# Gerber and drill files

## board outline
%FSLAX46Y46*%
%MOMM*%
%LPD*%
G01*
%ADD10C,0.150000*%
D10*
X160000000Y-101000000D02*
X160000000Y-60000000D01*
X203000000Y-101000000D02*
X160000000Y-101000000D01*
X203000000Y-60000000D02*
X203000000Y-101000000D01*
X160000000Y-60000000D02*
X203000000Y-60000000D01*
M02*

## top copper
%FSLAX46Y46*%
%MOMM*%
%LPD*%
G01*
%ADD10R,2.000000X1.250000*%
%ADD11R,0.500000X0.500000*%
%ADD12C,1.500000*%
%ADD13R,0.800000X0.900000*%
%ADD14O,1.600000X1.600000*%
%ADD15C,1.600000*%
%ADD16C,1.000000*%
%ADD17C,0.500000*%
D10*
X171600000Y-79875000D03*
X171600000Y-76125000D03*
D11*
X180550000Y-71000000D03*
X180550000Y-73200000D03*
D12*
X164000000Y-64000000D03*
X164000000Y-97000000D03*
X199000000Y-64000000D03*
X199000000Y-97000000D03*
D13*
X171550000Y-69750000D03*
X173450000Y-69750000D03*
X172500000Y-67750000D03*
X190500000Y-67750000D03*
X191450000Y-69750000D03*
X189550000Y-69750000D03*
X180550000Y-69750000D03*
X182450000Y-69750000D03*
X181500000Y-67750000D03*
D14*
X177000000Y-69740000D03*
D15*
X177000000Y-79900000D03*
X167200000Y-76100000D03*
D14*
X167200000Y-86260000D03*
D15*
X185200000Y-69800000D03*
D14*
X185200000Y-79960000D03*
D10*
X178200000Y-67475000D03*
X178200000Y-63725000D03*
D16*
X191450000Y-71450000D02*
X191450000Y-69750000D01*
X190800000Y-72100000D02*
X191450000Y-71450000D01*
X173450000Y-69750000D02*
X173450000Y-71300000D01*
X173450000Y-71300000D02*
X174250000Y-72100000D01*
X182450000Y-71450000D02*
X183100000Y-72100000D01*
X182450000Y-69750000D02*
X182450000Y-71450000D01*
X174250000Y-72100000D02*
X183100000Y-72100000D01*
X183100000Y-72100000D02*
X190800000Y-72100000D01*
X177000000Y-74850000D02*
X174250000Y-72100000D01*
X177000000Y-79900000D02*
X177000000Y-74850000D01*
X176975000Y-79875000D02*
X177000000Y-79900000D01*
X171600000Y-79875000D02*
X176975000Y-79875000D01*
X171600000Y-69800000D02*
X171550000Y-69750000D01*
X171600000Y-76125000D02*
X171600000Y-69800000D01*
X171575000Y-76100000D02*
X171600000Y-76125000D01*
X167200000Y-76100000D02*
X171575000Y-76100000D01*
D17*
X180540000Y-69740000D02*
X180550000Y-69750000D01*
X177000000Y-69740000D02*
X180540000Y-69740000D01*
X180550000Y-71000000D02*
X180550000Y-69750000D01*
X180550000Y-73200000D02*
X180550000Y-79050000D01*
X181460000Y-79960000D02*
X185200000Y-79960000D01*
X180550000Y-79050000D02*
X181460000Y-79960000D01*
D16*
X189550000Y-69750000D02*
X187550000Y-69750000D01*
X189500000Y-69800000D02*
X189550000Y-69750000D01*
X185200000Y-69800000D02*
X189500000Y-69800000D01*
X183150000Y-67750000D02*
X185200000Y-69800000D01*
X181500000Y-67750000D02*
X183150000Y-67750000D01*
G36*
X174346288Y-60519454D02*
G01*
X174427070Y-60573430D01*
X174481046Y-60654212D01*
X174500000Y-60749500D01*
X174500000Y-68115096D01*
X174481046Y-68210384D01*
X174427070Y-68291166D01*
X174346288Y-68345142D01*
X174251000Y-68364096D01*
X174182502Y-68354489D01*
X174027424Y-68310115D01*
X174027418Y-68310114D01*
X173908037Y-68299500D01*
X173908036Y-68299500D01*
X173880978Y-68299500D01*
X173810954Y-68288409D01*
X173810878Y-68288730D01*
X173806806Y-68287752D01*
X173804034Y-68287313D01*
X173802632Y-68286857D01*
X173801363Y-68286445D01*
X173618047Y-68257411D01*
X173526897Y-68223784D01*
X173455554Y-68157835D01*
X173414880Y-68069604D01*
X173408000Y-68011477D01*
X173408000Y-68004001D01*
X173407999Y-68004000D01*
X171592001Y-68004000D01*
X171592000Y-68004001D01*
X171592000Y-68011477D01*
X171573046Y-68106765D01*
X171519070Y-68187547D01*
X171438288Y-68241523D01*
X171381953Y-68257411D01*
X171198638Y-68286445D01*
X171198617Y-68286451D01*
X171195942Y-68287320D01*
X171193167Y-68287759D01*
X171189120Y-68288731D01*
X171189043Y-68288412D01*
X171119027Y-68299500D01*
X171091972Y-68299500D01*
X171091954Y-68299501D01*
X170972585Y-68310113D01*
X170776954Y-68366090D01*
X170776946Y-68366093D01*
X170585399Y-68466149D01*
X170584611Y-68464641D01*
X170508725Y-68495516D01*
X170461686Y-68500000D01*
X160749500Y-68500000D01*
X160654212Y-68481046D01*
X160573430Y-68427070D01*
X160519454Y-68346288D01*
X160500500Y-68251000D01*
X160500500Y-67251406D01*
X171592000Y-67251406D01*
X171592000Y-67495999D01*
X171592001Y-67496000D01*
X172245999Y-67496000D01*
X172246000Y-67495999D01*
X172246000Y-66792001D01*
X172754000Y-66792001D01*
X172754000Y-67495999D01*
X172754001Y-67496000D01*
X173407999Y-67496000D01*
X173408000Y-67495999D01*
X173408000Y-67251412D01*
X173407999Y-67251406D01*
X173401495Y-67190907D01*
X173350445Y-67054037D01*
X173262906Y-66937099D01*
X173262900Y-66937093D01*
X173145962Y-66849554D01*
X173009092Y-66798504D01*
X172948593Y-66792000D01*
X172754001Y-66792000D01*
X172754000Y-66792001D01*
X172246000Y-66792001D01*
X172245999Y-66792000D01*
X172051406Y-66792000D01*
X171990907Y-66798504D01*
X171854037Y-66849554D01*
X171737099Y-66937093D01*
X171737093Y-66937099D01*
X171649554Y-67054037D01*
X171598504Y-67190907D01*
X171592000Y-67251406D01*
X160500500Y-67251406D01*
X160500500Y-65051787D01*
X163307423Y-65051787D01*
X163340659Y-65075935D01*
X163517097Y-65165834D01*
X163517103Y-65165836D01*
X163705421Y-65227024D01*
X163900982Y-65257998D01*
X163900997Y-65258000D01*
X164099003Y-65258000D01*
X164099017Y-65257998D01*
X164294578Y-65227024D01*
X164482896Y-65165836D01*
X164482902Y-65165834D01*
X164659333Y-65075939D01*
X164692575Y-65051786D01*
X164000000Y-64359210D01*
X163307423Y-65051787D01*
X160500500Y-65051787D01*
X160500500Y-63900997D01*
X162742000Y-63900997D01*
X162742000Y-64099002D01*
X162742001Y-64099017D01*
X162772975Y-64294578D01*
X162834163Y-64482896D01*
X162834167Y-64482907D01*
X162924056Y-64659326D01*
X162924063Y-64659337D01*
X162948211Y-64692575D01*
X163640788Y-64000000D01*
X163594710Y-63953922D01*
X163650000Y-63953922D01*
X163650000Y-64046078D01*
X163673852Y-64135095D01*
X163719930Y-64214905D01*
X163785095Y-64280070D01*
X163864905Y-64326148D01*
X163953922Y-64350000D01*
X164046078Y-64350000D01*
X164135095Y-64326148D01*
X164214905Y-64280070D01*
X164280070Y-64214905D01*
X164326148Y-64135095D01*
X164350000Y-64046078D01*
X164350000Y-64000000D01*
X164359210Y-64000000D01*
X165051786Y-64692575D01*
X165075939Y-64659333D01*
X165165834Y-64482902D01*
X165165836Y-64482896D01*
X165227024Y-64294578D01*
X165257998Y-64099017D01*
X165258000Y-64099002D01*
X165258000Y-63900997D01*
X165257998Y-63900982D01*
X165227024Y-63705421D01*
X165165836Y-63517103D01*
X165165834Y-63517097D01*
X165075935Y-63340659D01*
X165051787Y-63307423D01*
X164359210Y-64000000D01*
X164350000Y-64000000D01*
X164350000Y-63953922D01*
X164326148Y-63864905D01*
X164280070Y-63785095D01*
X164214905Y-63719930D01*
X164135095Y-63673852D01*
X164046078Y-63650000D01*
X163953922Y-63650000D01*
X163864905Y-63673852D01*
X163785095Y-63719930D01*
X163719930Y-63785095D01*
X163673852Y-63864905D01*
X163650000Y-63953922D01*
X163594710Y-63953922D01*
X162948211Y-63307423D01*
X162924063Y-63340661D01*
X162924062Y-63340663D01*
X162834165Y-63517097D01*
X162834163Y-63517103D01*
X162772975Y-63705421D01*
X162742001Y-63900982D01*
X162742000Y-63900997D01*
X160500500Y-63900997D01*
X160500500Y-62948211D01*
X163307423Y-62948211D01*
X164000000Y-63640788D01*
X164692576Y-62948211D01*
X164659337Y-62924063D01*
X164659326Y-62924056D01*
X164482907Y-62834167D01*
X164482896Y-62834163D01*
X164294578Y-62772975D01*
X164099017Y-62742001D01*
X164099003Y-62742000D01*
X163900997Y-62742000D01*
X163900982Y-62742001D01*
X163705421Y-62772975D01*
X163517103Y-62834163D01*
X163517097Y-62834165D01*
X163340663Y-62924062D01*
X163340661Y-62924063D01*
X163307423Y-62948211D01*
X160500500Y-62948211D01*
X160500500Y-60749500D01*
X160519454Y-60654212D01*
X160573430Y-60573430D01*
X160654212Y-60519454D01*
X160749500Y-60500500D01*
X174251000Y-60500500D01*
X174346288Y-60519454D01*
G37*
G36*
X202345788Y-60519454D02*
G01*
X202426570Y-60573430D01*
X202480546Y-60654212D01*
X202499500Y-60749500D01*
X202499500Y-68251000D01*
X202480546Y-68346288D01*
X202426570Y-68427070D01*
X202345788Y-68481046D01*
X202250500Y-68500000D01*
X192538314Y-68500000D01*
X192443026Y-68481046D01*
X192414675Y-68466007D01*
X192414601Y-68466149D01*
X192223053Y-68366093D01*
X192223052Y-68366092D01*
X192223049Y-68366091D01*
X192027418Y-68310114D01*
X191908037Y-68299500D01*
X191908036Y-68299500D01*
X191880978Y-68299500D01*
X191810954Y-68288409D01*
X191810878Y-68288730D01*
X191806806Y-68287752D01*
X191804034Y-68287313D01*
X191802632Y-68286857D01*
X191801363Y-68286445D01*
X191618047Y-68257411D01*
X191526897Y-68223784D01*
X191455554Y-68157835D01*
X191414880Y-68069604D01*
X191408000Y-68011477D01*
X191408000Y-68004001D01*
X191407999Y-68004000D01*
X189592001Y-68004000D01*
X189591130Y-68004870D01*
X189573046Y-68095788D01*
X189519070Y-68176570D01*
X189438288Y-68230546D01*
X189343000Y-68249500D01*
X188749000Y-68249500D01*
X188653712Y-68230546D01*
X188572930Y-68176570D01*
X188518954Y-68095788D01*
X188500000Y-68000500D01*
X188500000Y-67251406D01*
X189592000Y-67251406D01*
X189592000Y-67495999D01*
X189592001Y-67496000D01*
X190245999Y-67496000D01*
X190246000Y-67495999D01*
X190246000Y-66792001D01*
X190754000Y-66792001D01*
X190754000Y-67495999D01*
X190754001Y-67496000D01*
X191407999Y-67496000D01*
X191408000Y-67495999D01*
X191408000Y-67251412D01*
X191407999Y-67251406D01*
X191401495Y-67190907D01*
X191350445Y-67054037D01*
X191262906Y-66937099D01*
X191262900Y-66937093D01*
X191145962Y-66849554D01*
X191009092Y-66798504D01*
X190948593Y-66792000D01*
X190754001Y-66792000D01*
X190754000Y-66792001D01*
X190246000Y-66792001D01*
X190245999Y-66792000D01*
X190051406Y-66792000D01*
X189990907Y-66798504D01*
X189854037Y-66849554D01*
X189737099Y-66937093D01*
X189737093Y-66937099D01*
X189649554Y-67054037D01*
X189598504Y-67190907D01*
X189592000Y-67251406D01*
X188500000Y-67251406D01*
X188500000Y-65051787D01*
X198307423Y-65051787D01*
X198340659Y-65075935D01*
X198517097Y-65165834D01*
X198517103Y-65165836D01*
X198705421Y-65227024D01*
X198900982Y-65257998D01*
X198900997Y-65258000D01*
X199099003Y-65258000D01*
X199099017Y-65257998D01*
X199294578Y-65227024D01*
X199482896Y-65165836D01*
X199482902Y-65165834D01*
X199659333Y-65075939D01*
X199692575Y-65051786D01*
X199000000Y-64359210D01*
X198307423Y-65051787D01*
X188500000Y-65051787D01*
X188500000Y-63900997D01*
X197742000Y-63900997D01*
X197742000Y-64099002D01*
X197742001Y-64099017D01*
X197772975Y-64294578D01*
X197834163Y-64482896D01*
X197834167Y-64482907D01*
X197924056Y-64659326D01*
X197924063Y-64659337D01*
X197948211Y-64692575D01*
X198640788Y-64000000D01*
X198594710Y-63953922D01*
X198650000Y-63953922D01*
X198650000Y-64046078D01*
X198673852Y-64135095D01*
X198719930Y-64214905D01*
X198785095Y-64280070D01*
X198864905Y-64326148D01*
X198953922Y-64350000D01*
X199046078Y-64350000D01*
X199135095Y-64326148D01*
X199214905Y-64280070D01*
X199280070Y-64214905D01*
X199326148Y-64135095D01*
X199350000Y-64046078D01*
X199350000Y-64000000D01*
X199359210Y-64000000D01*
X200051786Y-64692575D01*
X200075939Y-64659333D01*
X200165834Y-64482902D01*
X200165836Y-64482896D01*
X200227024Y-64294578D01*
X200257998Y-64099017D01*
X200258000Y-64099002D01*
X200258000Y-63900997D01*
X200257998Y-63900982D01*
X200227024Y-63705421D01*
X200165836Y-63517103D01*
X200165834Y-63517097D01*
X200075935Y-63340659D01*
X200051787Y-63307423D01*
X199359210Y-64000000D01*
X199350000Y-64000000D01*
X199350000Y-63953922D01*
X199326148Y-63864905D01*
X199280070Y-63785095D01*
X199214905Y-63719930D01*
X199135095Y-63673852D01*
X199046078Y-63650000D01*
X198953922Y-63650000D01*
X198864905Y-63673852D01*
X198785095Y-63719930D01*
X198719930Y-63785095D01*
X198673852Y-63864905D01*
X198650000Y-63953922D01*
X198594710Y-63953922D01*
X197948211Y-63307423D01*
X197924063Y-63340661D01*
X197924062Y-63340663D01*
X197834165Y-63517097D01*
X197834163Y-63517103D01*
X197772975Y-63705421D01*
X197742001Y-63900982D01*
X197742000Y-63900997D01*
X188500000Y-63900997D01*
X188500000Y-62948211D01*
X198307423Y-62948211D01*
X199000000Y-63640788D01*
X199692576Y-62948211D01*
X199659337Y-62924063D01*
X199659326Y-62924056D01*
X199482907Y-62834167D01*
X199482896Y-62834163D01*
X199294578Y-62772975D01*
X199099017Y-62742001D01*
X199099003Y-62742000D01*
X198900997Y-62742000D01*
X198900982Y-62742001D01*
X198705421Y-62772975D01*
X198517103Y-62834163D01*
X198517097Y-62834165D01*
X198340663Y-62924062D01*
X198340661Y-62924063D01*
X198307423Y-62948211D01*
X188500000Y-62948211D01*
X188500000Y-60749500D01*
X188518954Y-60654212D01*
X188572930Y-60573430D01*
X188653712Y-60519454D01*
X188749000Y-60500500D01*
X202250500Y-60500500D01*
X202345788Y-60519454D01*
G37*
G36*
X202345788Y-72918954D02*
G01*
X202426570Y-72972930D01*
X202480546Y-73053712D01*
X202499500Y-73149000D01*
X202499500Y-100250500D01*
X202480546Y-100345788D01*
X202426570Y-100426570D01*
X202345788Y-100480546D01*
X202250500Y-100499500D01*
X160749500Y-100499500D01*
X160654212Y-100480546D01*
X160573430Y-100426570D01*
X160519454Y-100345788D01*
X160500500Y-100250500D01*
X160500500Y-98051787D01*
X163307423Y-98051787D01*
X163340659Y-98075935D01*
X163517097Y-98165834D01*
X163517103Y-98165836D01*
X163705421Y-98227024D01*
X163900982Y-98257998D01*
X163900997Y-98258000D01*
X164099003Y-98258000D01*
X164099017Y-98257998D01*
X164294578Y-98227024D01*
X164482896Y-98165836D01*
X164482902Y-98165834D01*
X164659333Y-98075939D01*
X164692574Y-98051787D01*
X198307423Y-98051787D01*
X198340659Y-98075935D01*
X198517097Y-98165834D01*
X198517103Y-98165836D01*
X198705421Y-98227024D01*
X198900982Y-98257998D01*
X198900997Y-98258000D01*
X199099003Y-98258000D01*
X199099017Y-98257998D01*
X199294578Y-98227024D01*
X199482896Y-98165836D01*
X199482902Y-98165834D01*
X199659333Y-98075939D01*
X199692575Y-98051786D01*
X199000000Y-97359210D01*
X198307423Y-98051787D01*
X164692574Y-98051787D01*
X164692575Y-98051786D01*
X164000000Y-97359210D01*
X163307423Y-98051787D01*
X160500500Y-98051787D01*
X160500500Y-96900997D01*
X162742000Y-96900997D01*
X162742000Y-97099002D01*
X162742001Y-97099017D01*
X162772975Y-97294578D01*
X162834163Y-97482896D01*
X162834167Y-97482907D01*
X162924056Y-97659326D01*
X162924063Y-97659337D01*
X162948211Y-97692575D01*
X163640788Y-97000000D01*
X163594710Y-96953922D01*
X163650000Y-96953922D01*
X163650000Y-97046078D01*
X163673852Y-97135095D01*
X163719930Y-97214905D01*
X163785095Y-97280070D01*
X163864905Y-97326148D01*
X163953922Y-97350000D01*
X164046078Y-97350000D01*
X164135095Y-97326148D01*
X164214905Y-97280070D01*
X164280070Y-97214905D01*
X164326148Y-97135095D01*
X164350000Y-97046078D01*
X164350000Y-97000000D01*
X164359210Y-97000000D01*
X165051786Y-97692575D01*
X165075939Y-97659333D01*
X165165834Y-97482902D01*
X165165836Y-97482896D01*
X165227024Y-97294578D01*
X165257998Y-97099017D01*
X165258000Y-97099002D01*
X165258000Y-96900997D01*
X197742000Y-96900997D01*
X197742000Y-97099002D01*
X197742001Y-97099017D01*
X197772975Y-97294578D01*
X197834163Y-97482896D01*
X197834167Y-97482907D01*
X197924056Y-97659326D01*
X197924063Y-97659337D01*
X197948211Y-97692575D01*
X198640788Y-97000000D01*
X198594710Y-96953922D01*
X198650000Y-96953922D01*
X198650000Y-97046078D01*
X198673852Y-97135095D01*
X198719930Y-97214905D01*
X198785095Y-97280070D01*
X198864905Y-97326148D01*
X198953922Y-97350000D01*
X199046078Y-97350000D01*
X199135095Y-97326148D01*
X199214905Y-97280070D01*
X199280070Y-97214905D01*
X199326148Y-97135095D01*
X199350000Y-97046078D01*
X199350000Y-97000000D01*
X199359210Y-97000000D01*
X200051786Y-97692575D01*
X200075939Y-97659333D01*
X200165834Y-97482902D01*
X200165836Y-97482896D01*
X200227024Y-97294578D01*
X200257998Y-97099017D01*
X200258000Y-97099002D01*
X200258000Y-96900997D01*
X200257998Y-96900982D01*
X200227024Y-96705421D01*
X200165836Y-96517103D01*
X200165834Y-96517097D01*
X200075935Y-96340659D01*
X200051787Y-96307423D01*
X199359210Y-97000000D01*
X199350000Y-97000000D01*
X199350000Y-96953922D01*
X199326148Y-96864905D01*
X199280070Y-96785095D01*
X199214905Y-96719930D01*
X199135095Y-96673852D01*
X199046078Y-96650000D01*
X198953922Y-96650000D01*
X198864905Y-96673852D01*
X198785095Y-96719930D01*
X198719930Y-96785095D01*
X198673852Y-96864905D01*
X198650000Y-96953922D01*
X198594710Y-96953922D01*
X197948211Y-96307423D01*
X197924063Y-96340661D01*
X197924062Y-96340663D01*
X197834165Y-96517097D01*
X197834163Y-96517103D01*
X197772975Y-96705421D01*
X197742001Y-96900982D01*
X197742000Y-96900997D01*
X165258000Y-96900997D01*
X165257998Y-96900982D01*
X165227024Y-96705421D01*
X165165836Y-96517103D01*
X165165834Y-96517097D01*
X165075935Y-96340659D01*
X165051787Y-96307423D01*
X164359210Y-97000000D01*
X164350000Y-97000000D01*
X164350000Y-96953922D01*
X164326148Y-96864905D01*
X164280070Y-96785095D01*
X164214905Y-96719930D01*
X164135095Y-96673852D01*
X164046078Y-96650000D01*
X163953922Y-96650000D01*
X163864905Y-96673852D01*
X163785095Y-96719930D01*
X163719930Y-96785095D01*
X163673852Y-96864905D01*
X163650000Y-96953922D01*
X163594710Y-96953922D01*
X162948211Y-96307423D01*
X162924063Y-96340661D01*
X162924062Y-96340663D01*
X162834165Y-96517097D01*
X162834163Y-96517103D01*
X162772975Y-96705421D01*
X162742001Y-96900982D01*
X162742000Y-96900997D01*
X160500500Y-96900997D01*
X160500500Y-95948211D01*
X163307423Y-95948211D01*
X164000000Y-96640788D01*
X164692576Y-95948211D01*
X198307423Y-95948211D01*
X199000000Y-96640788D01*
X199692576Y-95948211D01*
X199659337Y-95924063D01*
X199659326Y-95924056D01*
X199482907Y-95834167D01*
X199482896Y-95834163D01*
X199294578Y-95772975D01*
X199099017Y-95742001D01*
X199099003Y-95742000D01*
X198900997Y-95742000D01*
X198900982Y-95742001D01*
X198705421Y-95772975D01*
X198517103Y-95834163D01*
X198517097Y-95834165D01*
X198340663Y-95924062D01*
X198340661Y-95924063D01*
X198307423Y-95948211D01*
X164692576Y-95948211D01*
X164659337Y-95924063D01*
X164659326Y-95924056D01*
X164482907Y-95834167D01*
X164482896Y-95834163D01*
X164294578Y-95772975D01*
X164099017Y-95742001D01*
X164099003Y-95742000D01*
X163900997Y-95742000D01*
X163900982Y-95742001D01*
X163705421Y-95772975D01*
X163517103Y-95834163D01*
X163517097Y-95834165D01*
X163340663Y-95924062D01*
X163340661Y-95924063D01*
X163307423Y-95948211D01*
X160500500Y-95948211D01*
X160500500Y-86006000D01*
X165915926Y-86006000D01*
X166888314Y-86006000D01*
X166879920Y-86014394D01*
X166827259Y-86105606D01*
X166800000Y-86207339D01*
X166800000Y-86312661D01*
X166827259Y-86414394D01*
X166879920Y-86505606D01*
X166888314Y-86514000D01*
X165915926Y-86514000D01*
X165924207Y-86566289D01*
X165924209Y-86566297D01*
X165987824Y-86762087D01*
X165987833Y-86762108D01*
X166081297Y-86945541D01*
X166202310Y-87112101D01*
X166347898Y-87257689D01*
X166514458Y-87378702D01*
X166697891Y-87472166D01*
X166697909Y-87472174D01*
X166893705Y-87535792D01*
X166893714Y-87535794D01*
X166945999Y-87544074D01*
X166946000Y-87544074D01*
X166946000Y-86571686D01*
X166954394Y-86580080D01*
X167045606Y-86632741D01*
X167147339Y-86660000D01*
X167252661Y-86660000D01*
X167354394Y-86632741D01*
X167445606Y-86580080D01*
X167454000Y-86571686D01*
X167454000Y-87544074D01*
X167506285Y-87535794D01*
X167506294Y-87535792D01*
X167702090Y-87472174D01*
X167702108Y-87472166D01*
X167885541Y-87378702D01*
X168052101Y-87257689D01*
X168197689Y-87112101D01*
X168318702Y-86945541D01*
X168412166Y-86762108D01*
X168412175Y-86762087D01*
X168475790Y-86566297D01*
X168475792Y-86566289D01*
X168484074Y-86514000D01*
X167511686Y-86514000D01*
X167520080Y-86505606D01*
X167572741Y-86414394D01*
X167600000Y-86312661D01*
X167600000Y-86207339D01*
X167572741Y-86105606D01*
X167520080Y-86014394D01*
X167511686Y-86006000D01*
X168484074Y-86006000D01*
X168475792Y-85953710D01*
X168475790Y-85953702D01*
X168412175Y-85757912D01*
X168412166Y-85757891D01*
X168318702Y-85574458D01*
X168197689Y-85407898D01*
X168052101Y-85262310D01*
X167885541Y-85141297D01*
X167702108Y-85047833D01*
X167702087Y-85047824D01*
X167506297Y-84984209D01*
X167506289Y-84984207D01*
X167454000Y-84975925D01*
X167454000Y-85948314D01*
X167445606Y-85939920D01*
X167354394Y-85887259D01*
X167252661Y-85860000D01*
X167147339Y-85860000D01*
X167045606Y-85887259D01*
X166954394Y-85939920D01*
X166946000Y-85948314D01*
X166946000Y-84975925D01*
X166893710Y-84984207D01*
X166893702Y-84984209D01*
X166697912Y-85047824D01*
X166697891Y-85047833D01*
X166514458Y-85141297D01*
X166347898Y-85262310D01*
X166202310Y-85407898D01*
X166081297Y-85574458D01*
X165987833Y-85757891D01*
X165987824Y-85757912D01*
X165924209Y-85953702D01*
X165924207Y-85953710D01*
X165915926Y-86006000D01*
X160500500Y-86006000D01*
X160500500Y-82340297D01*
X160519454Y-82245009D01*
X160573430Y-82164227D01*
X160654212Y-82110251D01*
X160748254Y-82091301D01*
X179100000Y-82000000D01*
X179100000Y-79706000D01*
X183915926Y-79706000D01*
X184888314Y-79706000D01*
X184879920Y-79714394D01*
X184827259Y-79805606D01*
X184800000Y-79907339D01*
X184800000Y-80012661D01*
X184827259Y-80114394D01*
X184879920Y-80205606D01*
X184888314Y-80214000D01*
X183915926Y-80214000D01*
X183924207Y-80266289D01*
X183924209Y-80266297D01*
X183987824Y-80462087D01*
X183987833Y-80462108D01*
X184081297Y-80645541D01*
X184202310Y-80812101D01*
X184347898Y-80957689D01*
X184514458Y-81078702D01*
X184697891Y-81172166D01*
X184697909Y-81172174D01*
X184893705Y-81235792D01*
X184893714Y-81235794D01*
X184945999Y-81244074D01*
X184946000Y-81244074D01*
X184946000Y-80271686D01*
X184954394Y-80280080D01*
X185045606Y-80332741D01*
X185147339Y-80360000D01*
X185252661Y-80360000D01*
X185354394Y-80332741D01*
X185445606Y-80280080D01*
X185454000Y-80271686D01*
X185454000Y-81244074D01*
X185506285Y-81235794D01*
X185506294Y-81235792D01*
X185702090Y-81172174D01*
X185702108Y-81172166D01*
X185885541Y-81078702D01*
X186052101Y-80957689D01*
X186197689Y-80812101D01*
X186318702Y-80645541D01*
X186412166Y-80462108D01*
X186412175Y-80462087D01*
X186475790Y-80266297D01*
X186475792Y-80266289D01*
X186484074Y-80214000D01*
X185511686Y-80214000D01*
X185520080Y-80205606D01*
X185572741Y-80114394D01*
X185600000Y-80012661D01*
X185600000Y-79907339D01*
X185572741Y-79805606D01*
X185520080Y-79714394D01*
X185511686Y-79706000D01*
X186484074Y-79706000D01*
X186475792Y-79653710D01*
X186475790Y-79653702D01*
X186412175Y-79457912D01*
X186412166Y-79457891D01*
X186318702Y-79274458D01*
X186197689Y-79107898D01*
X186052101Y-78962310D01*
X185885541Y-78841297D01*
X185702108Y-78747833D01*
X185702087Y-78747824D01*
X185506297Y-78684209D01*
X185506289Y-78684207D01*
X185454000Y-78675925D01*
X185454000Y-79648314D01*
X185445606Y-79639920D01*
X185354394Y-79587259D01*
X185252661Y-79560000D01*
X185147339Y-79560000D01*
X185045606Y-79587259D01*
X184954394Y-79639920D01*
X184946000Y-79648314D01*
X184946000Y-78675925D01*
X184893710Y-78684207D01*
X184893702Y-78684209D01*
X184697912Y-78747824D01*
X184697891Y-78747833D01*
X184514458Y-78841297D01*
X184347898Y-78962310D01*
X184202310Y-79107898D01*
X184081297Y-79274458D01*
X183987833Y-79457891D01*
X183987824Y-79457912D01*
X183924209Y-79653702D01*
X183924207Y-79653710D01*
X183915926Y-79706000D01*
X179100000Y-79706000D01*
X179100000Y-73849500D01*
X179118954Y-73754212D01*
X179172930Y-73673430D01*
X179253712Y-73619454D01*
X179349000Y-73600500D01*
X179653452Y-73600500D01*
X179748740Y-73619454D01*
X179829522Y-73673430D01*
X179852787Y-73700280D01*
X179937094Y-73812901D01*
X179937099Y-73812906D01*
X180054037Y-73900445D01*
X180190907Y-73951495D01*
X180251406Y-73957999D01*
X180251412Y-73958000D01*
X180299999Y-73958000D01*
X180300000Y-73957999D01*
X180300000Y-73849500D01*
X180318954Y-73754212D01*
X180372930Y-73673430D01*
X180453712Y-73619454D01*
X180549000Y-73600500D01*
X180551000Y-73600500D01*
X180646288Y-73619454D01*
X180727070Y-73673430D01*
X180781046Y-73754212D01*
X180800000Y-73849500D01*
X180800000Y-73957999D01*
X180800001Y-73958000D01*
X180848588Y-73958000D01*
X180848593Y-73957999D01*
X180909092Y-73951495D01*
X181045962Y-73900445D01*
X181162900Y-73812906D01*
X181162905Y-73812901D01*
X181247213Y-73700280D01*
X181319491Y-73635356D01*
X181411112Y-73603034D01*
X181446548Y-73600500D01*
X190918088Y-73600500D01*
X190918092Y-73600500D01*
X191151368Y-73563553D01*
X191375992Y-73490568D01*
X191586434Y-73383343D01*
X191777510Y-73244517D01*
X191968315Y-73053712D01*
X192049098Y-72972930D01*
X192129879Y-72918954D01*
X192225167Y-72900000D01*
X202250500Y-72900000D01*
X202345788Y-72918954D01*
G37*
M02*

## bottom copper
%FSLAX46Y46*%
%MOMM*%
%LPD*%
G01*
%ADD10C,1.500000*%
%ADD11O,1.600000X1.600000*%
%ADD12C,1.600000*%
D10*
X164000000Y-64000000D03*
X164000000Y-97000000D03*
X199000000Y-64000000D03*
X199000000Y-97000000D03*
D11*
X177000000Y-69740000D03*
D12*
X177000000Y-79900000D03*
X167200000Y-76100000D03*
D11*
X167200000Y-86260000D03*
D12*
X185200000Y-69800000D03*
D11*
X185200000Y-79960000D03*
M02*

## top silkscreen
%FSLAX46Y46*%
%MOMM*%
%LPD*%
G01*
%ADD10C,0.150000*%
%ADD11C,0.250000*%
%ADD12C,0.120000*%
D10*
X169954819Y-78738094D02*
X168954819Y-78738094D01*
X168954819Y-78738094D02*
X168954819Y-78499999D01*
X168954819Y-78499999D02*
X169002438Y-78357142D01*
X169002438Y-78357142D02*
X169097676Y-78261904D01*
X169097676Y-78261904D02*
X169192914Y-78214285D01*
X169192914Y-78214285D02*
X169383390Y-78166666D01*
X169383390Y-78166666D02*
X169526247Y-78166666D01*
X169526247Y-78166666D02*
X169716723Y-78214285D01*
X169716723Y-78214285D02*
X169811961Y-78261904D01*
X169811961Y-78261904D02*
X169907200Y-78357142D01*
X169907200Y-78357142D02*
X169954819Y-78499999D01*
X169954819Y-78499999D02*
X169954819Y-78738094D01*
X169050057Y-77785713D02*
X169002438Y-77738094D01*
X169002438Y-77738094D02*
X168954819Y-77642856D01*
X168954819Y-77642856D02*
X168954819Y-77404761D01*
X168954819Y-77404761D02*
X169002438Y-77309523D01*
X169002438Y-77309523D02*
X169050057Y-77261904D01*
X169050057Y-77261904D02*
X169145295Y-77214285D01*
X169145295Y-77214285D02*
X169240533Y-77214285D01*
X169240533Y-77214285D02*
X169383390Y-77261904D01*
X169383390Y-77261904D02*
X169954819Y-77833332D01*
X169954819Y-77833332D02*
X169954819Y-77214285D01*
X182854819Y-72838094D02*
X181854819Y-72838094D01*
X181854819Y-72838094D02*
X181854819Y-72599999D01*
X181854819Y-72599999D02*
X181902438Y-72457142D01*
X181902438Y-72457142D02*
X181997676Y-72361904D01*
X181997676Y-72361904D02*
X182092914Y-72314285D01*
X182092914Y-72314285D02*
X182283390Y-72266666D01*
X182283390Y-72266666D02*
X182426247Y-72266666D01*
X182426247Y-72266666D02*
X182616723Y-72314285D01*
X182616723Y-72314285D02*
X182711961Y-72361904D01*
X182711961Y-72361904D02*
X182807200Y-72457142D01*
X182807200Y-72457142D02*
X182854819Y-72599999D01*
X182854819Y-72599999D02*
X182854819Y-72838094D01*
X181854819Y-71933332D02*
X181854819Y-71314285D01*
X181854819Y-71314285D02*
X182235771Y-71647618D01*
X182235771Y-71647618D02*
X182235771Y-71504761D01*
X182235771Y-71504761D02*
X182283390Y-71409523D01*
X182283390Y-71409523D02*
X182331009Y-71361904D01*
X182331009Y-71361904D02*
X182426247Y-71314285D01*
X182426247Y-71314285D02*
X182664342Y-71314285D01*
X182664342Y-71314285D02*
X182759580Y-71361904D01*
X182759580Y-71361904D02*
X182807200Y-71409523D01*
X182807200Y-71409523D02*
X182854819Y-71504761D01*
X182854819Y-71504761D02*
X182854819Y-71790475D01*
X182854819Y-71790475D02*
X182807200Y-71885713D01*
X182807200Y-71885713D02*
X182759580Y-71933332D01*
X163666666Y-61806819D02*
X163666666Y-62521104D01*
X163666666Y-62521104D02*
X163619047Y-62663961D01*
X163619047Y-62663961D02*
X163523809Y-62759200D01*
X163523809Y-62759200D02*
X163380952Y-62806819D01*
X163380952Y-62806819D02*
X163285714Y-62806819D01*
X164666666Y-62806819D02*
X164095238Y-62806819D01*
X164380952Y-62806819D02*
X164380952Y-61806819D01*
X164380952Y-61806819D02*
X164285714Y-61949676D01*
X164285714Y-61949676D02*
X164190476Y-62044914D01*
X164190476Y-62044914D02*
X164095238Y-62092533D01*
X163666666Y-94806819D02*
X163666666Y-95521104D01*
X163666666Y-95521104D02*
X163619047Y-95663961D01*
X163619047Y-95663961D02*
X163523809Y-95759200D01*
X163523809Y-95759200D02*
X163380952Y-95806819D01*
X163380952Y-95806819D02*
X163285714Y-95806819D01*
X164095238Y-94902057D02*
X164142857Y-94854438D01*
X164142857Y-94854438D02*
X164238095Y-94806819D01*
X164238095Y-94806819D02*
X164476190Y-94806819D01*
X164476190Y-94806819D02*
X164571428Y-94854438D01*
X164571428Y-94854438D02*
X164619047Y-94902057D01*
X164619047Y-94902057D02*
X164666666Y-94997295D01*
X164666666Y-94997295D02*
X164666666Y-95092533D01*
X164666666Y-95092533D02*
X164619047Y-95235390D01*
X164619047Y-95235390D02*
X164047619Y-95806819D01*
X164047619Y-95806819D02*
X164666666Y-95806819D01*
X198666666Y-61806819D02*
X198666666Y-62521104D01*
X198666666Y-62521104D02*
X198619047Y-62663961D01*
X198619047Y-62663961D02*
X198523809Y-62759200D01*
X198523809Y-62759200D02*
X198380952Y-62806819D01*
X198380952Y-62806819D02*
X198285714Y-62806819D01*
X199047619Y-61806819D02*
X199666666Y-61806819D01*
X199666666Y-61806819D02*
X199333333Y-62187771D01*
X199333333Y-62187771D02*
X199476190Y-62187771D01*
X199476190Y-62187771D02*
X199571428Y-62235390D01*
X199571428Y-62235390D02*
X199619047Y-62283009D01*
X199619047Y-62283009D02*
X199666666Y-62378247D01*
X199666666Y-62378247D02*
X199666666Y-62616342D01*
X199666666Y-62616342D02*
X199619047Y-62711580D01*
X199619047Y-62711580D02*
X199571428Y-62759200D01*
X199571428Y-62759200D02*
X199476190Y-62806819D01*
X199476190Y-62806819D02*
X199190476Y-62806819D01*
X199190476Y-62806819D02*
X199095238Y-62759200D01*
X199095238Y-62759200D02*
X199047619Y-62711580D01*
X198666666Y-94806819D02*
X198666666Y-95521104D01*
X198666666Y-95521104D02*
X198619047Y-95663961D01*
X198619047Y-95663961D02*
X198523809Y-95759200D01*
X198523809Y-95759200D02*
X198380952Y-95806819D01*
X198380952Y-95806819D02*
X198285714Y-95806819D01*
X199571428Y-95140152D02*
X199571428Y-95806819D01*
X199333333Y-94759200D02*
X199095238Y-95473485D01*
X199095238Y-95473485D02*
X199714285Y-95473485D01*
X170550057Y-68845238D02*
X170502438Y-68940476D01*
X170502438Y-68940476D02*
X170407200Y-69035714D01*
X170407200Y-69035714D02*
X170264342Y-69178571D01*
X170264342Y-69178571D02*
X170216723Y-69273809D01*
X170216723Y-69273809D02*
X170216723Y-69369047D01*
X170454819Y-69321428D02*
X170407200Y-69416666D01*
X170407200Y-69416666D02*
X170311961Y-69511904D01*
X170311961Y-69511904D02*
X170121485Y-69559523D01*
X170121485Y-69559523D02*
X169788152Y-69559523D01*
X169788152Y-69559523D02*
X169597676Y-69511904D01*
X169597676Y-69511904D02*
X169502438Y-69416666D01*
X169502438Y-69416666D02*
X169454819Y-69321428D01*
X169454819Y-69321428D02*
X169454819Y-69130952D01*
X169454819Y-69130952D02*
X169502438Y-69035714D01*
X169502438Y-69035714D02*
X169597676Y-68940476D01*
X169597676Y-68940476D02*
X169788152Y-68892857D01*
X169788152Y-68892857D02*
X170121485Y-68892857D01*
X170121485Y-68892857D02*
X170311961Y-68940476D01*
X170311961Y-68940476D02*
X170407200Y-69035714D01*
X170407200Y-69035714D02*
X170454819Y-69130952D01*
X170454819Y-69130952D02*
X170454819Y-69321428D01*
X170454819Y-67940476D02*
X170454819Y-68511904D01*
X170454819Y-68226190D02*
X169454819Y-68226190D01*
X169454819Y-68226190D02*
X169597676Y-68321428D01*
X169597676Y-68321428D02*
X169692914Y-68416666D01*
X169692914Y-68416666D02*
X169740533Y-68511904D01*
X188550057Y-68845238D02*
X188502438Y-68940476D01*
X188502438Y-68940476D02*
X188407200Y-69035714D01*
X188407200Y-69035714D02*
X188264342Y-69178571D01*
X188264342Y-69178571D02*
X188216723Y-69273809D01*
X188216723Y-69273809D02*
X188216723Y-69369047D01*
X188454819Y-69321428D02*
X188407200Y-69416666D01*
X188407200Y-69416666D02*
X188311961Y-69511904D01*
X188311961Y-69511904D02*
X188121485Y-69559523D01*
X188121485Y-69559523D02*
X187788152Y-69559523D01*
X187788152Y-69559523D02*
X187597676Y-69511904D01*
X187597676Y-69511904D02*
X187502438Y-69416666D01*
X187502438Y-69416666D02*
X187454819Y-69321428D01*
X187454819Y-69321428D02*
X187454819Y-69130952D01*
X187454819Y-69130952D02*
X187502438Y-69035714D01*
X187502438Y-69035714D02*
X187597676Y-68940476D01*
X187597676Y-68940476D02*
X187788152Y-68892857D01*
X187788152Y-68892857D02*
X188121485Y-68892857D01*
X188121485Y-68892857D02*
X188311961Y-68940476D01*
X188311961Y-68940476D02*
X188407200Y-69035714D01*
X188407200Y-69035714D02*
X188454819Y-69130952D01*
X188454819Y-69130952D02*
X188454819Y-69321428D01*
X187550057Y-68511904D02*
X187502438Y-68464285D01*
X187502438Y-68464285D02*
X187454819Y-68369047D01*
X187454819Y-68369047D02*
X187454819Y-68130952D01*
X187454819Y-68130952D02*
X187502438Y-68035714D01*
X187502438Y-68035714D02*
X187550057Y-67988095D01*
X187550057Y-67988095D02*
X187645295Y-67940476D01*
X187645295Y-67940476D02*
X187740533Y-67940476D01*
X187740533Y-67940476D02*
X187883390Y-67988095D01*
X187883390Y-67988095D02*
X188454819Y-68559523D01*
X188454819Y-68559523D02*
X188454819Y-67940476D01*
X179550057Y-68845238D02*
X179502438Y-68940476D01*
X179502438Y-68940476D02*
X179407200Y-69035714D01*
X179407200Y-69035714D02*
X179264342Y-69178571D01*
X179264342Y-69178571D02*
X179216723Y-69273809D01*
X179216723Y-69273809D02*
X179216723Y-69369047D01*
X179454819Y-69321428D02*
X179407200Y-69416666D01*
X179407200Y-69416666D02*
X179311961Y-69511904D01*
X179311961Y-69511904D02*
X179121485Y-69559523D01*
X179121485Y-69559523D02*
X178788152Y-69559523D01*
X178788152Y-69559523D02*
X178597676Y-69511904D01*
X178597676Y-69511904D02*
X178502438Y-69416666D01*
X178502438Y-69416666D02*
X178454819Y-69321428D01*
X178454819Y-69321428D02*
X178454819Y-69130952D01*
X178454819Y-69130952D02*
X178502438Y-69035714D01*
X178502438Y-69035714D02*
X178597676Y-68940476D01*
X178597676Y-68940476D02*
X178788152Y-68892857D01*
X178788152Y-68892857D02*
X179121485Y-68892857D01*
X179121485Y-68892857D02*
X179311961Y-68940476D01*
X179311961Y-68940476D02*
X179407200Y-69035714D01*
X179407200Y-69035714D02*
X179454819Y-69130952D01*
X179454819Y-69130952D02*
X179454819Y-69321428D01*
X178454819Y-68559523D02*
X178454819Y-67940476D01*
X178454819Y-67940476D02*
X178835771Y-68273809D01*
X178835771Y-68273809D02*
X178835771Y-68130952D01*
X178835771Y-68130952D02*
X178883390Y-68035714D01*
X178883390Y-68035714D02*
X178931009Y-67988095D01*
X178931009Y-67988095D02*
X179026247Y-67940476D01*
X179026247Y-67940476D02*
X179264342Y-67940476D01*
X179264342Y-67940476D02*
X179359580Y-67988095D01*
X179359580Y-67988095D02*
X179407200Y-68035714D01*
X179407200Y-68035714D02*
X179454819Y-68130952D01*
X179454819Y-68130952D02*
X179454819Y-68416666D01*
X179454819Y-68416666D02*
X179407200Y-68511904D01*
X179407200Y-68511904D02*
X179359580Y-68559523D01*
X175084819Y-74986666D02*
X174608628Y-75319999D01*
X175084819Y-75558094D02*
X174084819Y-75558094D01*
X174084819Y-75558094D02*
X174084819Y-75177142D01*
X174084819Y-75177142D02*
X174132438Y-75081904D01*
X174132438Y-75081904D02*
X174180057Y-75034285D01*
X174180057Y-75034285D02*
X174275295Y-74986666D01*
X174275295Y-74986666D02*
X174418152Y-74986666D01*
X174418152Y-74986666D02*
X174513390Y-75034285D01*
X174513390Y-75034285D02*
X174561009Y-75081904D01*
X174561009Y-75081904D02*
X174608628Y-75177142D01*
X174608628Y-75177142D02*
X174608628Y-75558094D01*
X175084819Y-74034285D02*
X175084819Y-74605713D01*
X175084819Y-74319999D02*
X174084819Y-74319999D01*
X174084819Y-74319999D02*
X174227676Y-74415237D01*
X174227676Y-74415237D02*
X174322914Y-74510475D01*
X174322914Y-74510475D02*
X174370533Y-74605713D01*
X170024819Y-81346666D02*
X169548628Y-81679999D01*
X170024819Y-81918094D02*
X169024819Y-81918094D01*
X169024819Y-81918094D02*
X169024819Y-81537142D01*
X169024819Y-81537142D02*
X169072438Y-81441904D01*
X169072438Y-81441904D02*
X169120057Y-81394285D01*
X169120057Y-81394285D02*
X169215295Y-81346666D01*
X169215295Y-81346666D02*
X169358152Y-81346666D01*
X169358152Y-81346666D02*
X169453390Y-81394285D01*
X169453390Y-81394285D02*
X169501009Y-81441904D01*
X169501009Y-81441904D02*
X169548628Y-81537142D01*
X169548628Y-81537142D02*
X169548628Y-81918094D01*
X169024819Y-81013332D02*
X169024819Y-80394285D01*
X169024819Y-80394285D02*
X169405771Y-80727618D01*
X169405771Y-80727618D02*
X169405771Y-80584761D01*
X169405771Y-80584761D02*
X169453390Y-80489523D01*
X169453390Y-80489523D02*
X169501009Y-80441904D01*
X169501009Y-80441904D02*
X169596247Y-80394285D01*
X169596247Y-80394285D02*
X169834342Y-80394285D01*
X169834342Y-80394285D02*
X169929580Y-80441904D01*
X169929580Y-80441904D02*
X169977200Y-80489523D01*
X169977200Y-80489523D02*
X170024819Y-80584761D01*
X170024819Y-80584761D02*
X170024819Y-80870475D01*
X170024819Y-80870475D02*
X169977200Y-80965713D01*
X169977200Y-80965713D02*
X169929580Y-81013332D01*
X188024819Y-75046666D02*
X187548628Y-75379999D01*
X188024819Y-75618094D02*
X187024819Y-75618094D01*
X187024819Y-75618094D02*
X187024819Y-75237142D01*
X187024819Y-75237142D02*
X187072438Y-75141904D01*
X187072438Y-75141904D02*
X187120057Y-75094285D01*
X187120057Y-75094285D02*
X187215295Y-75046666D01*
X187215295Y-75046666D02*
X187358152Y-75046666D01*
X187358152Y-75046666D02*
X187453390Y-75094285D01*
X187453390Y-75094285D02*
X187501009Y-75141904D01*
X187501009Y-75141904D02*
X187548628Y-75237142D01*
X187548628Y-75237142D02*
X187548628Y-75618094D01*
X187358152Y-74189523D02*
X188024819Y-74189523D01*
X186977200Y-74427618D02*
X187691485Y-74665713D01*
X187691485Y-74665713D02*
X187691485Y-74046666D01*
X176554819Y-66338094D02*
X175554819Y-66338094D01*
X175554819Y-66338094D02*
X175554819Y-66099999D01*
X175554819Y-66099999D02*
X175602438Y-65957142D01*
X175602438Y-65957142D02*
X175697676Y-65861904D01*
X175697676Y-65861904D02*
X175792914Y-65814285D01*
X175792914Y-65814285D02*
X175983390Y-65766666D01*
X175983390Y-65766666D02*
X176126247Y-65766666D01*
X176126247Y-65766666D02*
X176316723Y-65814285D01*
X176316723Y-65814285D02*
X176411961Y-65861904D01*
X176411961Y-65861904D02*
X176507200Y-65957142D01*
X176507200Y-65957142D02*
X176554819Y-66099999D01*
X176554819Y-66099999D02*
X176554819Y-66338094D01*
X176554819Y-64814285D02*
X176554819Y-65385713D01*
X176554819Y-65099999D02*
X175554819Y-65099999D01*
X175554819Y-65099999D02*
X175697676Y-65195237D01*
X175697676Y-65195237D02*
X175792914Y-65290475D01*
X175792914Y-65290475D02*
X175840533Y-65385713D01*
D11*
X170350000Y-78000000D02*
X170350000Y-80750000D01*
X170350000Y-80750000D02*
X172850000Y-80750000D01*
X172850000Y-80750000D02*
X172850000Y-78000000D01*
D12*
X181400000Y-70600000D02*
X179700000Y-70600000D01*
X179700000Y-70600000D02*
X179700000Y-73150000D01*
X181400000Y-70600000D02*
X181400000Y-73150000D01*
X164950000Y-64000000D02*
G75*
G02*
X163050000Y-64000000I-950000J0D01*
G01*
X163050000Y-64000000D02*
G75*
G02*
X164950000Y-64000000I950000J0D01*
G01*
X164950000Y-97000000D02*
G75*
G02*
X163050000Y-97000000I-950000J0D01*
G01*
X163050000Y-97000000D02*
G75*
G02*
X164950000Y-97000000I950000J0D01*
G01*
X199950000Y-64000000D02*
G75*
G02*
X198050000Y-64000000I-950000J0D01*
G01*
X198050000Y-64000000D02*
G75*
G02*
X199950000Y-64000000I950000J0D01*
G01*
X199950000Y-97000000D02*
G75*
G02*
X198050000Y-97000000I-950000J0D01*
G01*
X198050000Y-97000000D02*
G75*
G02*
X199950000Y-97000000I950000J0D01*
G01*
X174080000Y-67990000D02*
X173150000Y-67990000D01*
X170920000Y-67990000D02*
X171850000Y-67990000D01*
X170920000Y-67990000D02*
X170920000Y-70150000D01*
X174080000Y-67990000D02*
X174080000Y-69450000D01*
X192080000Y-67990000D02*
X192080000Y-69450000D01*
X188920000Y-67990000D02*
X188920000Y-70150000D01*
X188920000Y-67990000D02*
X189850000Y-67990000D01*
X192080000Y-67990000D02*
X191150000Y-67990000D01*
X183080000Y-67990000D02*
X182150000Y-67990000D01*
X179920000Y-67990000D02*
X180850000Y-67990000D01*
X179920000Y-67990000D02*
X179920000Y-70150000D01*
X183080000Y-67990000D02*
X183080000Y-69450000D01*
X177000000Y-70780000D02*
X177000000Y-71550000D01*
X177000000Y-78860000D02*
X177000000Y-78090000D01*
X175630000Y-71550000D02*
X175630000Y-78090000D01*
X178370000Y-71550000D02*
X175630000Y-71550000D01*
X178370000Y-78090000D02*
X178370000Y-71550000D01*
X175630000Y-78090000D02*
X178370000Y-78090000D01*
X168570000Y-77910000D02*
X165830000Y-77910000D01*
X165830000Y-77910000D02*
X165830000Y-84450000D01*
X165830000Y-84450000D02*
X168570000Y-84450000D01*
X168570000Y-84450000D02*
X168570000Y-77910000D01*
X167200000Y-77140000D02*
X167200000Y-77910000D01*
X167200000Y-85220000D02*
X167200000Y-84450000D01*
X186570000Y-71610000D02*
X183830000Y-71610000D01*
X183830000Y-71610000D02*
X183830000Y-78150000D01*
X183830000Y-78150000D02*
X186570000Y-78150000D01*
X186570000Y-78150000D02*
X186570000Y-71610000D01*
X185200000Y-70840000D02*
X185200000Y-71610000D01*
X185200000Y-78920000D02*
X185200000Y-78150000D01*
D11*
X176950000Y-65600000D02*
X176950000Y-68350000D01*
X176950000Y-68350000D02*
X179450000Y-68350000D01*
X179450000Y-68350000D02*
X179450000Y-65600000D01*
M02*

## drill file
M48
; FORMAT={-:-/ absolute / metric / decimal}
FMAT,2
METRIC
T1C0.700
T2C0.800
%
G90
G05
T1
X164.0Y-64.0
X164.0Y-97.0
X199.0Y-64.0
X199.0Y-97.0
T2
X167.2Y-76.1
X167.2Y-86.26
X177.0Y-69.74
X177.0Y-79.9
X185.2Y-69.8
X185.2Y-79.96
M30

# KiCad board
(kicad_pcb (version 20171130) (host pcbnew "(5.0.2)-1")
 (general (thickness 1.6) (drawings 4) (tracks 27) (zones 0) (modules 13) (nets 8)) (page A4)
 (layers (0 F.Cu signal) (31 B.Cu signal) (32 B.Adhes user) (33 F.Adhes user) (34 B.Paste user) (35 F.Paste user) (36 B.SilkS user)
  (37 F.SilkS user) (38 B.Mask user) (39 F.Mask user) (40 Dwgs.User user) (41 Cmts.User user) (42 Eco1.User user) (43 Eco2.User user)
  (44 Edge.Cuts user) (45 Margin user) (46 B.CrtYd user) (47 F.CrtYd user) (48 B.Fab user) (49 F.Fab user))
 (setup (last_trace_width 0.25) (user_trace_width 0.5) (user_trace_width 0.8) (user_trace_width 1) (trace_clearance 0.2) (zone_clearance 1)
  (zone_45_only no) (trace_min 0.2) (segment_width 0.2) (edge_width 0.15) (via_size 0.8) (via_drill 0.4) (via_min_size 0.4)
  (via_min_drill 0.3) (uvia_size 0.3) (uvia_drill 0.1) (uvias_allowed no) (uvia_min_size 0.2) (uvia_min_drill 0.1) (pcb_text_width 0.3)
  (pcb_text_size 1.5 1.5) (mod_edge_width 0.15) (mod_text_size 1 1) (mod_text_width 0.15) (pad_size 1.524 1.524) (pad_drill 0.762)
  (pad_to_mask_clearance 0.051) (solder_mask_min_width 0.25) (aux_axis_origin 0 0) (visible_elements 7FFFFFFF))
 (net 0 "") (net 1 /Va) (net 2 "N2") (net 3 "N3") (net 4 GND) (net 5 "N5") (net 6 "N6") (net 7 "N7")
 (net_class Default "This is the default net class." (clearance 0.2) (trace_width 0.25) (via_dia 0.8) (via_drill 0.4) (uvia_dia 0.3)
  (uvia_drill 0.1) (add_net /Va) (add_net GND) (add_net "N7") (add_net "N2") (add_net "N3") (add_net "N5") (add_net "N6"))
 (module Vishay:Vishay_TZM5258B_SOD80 (layer F.Cu) (at 171.6 78 90)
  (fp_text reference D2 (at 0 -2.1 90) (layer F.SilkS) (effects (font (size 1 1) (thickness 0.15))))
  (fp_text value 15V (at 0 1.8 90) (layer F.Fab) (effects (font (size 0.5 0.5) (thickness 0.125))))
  (fp_line (start 0 -1.25) (end -2.75 -1.25) (layer F.SilkS) (width 0.25))
  (fp_line (start -2.75 -1.25) (end -2.75 1.25) (layer F.SilkS) (width 0.25))
  (fp_line (start -2.75 1.25) (end 0 1.25) (layer F.SilkS) (width 0.25))
  (pad 1 smd rect (at -1.875 0 90) (size 1.25 2) (layers F.Cu F.Paste F.Mask) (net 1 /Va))
  (pad 2 smd rect (at 1.875 0 90) (size 1.25 2) (layers F.Cu F.Paste F.Mask) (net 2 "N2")))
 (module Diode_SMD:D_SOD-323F (layer F.Cu) (at 180.55 72.1 270)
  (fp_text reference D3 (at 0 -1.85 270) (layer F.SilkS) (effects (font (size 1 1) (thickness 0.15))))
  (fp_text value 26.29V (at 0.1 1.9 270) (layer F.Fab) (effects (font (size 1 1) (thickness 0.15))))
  (fp_line (start -1.5 -0.85) (end -1.5 0.85) (layer F.SilkS) (width 0.12))
  (fp_line (start -1.5 0.85) (end 1.05 0.85) (layer F.SilkS) (width 0.12))
  (fp_line (start -1.5 -0.85) (end 1.05 -0.85) (layer F.SilkS) (width 0.12))
  (pad 1 smd rect (at -1.1 0 270) (size 0.5 0.5) (layers F.Cu F.Paste F.Mask) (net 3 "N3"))
  (pad 2 smd rect (at 1.1 0 270) (size 0.5 0.5) (layers F.Cu F.Paste F.Mask) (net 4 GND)))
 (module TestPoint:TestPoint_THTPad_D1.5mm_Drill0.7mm (layer F.Cu) (at 164 64)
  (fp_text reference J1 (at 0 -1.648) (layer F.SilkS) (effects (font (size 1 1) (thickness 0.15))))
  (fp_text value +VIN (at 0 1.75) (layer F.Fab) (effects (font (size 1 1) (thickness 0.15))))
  (fp_circle (center 0 0) (end 0 0.95) (layer F.SilkS) (width 0.12))
  (pad 1 thru_hole circle (at 0 0) (size 1.5 1.5) (drill 0.7) (layers *.Cu *.Mask) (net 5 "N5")))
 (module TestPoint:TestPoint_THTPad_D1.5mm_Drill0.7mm (layer F.Cu) (at 164 97)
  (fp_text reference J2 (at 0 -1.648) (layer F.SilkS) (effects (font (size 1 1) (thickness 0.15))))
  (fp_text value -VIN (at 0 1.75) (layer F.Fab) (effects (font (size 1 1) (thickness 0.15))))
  (fp_circle (center 0 0) (end 0 0.95) (layer F.SilkS) (width 0.12))
  (pad 1 thru_hole circle (at 0 0) (size 1.5 1.5) (drill 0.7) (layers *.Cu *.Mask) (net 4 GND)))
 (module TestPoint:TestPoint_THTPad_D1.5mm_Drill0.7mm (layer F.Cu) (at 199 64)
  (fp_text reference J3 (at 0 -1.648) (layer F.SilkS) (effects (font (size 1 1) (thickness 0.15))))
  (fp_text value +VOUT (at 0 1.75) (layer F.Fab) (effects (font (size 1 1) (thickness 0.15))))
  (fp_circle (center 0 0) (end 0 0.95) (layer F.SilkS) (width 0.12))
  (pad 1 thru_hole circle (at 0 0) (size 1.5 1.5) (drill 0.7) (layers *.Cu *.Mask) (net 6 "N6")))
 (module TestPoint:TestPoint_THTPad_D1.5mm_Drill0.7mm (layer F.Cu) (at 199 97)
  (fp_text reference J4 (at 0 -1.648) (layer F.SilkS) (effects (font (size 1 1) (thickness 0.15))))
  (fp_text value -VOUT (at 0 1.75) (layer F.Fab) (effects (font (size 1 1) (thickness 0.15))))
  (fp_circle (center 0 0) (end 0 0.95) (layer F.SilkS) (width 0.12))
  (pad 1 thru_hole circle (at 0 0) (size 1.5 1.5) (drill 0.7) (layers *.Cu *.Mask) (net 4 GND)))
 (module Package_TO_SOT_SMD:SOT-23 (layer F.Cu) (at 172.5 68.75 90)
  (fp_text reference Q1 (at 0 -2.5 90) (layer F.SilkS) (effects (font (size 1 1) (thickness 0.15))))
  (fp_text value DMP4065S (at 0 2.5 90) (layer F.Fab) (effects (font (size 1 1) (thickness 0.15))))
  (fp_line (start 0.76 1.58) (end 0.76 0.65) (layer F.SilkS) (width 0.12))
  (fp_line (start 0.76 -1.58) (end 0.76 -0.65) (layer F.SilkS) (width 0.12))
  (fp_line (start 0.76 -1.58) (end -1.4 -1.58) (layer F.SilkS) (width 0.12))
  (fp_line (start 0.76 1.58) (end -0.7 1.58) (layer F.SilkS) (width 0.12))
  (pad 1 smd rect (at -1 -0.95 90) (size 0.9 0.8) (layers F.Cu F.Paste F.Mask) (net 2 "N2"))
  (pad 2 smd rect (at -1 0.95 90) (size 0.9 0.8) (layers F.Cu F.Paste F.Mask) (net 1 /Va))
  (pad 3 smd rect (at 1 0 90) (size 0.9 0.8) (layers F.Cu F.Paste F.Mask) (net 5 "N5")))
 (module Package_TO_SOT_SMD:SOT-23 (layer F.Cu) (at 190.5 68.75 90)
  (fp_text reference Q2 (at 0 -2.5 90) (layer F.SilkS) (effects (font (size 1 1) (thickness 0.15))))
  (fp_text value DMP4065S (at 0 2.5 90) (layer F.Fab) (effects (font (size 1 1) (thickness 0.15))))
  (fp_line (start 0.76 1.58) (end -0.7 1.58) (layer F.SilkS) (width 0.12))
  (fp_line (start 0.76 -1.58) (end -1.4 -1.58) (layer F.SilkS) (width 0.12))
  (fp_line (start 0.76 -1.58) (end 0.76 -0.65) (layer F.SilkS) (width 0.12))
  (fp_line (start 0.76 1.58) (end 0.76 0.65) (layer F.SilkS) (width 0.12))
  (pad 3 smd rect (at 1 0 90) (size 0.9 0.8) (layers F.Cu F.Paste F.Mask) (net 6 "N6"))
  (pad 2 smd rect (at -1 0.95 90) (size 0.9 0.8) (layers F.Cu F.Paste F.Mask) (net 1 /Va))
  (pad 1 smd rect (at -1 -0.95 90) (size 0.9 0.8) (layers F.Cu F.Paste F.Mask) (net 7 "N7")))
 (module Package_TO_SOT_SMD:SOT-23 (layer F.Cu) (at 181.5 68.75 90)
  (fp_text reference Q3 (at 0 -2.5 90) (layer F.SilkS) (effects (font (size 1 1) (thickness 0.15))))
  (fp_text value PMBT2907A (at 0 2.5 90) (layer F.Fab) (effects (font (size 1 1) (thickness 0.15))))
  (fp_line (start 0.76 1.58) (end 0.76 0.65) (layer F.SilkS) (width 0.12))
  (fp_line (start 0.76 -1.58) (end 0.76 -0.65) (layer F.SilkS) (width 0.12))
  (fp_line (start 0.76 -1.58) (end -1.4 -1.58) (layer F.SilkS) (width 0.12))
  (fp_line (start 0.76 1.58) (end -0.7 1.58) (layer F.SilkS) (width 0.12))
  (pad 1 smd rect (at -1 -0.95 90) (size 0.9 0.8) (layers F.Cu F.Paste F.Mask) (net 3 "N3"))
  (pad 2 smd rect (at -1 0.95 90) (size 0.9 0.8) (layers F.Cu F.Paste F.Mask) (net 1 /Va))
  (pad 3 smd rect (at 1 0 90) (size 0.9 0.8) (layers F.Cu F.Paste F.Mask) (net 7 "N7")))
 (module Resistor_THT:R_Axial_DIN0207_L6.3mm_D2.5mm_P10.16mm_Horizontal (layer F.Cu) (at 177 79.9 90)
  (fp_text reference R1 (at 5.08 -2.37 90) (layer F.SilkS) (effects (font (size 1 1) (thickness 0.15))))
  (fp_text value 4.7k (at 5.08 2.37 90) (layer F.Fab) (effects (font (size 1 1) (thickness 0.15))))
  (fp_line (start 9.12 0) (end 8.35 0) (layer F.SilkS) (width 0.12))
  (fp_line (start 1.04 0) (end 1.81 0) (layer F.SilkS) (width 0.12))
  (fp_line (start 8.35 -1.37) (end 1.81 -1.37) (layer F.SilkS) (width 0.12))
  (fp_line (start 8.35 1.37) (end 8.35 -1.37) (layer F.SilkS) (width 0.12))
  (fp_line (start 1.81 1.37) (end 8.35 1.37) (layer F.SilkS) (width 0.12))
  (fp_line (start 1.81 -1.37) (end 1.81 1.37) (layer F.SilkS) (width 0.12))
  (pad 2 thru_hole oval (at 10.16 0 90) (size 1.6 1.6) (drill 0.8) (layers *.Cu *.Mask) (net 3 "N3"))
  (pad 1 thru_hole circle (at 0 0 90) (size 1.6 1.6) (drill 0.8) (layers *.Cu *.Mask) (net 1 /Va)))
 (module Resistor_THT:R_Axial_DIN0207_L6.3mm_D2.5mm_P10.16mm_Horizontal (layer F.Cu) (at 167.2 76.1 270)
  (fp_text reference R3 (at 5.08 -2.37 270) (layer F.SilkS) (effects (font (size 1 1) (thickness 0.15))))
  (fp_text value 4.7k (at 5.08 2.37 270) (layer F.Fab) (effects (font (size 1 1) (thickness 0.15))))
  (fp_line (start 1.81 -1.37) (end 1.81 1.37) (layer F.SilkS) (width 0.12))
  (fp_line (start 1.81 1.37) (end 8.35 1.37) (layer F.SilkS) (width 0.12))
  (fp_line (start 8.35 1.37) (end 8.35 -1.37) (layer F.SilkS) (width 0.12))
  (fp_line (start 8.35 -1.37) (end 1.81 -1.37) (layer F.SilkS) (width 0.12))
  (fp_line (start 1.04 0) (end 1.81 0) (layer F.SilkS) (width 0.12))
  (fp_line (start 9.12 0) (end 8.35 0) (layer F.SilkS) (width 0.12))
  (pad 1 thru_hole circle (at 0 0 270) (size 1.6 1.6) (drill 0.8) (layers *.Cu *.Mask) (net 2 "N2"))
  (pad 2 thru_hole oval (at 10.16 0 270) (size 1.6 1.6) (drill 0.8) (layers *.Cu *.Mask) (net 4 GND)))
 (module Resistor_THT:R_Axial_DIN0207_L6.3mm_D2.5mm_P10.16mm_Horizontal (layer F.Cu) (at 185.2 69.8 270)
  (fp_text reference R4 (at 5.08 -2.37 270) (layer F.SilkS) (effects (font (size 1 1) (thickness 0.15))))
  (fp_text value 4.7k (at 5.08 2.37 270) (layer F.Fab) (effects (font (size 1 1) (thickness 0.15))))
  (fp_line (start 1.81 -1.37) (end 1.81 1.37) (layer F.SilkS) (width 0.12))
  (fp_line (start 1.81 1.37) (end 8.35 1.37) (layer F.SilkS) (width 0.12))
  (fp_line (start 8.35 1.37) (end 8.35 -1.37) (layer F.SilkS) (width 0.12))
  (fp_line (start 8.35 -1.37) (end 1.81 -1.37) (layer F.SilkS) (width 0.12))
  (fp_line (start 1.04 0) (end 1.81 0) (layer F.SilkS) (width 0.12))
  (fp_line (start 9.12 0) (end 8.35 0) (layer F.SilkS) (width 0.12))
  (pad 1 thru_hole circle (at 0 0 270) (size 1.6 1.6) (drill 0.8) (layers *.Cu *.Mask) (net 7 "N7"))
  (pad 2 thru_hole oval (at 10.16 0 270) (size 1.6 1.6) (drill 0.8) (layers *.Cu *.Mask) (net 4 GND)))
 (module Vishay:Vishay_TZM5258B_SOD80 (layer F.Cu) (at 178.2 65.6 90)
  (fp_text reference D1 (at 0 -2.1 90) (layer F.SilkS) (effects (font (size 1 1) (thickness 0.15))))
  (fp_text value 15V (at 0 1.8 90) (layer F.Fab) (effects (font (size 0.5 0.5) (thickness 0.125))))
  (fp_line (start 0 -1.25) (end -2.75 -1.25) (layer F.SilkS) (width 0.25))
  (fp_line (start -2.75 -1.25) (end -2.75 1.25) (layer F.SilkS) (width 0.25))
  (fp_line (start -2.75 1.25) (end 0 1.25) (layer F.SilkS) (width 0.25))
  (pad 1 smd rect (at -1.875 0 90) (size 1.25 2) (layers F.Cu F.Paste F.Mask) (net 1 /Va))
  (pad 2 smd rect (at 1.875 0 90) (size 1.25 2) (layers F.Cu F.Paste F.Mask) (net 7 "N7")))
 (gr_line (start 160 101) (end 160 60) (layer Edge.Cuts) (width 0.15))
 (gr_line (start 203 101) (end 160 101) (layer Edge.Cuts) (width 0.15))
 (gr_line (start 203 60) (end 203 101) (layer Edge.Cuts) (width 0.15))
 (gr_line (start 160 60) (end 203 60) (layer Edge.Cuts) (width 0.15))
 (segment (start 191.45 71.45) (end 191.45 69.75) (width 1) (layer F.Cu) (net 1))
 (segment (start 190.8 72.1) (end 191.45 71.45) (width 1) (layer F.Cu) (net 1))
 (segment (start 173.45 69.75) (end 173.45 71.3) (width 1) (layer F.Cu) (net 1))
 (segment (start 173.45 71.3) (end 174.25 72.1) (width 1) (layer F.Cu) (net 1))
 (segment (start 182.45 71.45) (end 183.1 72.1) (width 1) (layer F.Cu) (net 1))
 (segment (start 182.45 69.75) (end 182.45 71.45) (width 1) (layer F.Cu) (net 1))
 (segment (start 174.25 72.1) (end 183.1 72.1) (width 1) (layer F.Cu) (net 1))
 (segment (start 183.1 72.1) (end 190.8 72.1) (width 1) (layer F.Cu) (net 1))
 (segment (start 177 74.85) (end 174.25 72.1) (width 1) (layer F.Cu) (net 1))
 (segment (start 177 79.9) (end 177 74.85) (width 1) (layer F.Cu) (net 1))
 (segment (start 176.975 79.875) (end 177 79.9) (width 1) (layer F.Cu) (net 1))
 (segment (start 171.6 79.875) (end 176.975 79.875) (width 1) (layer F.Cu) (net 1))
 (segment (start 171.6 69.8) (end 171.55 69.75) (width 1) (layer F.Cu) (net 2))
 (segment (start 171.6 76.125) (end 171.6 69.8) (width 1) (layer F.Cu) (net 2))
 (segment (start 171.575 76.1) (end 171.6 76.125) (width 1) (layer F.Cu) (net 2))
 (segment (start 167.2 76.1) (end 171.575 76.1) (width 1) (layer F.Cu) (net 2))
 (segment (start 180.54 69.74) (end 180.55 69.75) (width 0.5) (layer F.Cu) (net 3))
 (segment (start 177 69.74) (end 180.54 69.74) (width 0.5) (layer F.Cu) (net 3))
 (segment (start 180.55 71) (end 180.55 69.75) (width 0.5) (layer F.Cu) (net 3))
 (segment (start 180.55 73.2) (end 180.55 79.05) (width 0.5) (layer F.Cu) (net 4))
 (segment (start 181.46 79.96) (end 185.2 79.96) (width 0.5) (layer F.Cu) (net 4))
 (segment (start 180.55 79.05) (end 181.46 79.96) (width 0.5) (layer F.Cu) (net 4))
 (segment (start 189.55 69.75) (end 187.55 69.75) (width 1) (layer F.Cu) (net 7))
 (segment (start 189.5 69.8) (end 189.55 69.75) (width 1) (layer F.Cu) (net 7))
 (segment (start 185.2 69.8) (end 189.5 69.8) (width 1) (layer F.Cu) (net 7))
 (segment (start 183.15 67.75) (end 185.2 69.8) (width 1) (layer F.Cu) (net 7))
 (segment (start 181.5 67.75) (end 183.15 67.75) (width 1) (layer F.Cu) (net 7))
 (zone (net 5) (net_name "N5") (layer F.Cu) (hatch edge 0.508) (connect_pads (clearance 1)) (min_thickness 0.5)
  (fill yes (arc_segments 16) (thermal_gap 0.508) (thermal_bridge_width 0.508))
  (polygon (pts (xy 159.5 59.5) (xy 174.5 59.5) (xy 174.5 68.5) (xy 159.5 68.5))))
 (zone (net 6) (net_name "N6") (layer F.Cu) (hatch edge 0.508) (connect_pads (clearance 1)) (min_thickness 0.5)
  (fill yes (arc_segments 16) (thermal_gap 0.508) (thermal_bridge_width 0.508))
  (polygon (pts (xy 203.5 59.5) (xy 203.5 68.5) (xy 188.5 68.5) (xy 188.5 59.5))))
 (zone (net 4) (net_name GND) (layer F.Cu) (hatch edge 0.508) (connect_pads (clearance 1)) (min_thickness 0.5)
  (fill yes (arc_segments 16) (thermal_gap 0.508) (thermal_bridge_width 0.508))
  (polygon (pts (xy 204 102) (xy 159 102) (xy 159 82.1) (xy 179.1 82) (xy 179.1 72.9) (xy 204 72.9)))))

